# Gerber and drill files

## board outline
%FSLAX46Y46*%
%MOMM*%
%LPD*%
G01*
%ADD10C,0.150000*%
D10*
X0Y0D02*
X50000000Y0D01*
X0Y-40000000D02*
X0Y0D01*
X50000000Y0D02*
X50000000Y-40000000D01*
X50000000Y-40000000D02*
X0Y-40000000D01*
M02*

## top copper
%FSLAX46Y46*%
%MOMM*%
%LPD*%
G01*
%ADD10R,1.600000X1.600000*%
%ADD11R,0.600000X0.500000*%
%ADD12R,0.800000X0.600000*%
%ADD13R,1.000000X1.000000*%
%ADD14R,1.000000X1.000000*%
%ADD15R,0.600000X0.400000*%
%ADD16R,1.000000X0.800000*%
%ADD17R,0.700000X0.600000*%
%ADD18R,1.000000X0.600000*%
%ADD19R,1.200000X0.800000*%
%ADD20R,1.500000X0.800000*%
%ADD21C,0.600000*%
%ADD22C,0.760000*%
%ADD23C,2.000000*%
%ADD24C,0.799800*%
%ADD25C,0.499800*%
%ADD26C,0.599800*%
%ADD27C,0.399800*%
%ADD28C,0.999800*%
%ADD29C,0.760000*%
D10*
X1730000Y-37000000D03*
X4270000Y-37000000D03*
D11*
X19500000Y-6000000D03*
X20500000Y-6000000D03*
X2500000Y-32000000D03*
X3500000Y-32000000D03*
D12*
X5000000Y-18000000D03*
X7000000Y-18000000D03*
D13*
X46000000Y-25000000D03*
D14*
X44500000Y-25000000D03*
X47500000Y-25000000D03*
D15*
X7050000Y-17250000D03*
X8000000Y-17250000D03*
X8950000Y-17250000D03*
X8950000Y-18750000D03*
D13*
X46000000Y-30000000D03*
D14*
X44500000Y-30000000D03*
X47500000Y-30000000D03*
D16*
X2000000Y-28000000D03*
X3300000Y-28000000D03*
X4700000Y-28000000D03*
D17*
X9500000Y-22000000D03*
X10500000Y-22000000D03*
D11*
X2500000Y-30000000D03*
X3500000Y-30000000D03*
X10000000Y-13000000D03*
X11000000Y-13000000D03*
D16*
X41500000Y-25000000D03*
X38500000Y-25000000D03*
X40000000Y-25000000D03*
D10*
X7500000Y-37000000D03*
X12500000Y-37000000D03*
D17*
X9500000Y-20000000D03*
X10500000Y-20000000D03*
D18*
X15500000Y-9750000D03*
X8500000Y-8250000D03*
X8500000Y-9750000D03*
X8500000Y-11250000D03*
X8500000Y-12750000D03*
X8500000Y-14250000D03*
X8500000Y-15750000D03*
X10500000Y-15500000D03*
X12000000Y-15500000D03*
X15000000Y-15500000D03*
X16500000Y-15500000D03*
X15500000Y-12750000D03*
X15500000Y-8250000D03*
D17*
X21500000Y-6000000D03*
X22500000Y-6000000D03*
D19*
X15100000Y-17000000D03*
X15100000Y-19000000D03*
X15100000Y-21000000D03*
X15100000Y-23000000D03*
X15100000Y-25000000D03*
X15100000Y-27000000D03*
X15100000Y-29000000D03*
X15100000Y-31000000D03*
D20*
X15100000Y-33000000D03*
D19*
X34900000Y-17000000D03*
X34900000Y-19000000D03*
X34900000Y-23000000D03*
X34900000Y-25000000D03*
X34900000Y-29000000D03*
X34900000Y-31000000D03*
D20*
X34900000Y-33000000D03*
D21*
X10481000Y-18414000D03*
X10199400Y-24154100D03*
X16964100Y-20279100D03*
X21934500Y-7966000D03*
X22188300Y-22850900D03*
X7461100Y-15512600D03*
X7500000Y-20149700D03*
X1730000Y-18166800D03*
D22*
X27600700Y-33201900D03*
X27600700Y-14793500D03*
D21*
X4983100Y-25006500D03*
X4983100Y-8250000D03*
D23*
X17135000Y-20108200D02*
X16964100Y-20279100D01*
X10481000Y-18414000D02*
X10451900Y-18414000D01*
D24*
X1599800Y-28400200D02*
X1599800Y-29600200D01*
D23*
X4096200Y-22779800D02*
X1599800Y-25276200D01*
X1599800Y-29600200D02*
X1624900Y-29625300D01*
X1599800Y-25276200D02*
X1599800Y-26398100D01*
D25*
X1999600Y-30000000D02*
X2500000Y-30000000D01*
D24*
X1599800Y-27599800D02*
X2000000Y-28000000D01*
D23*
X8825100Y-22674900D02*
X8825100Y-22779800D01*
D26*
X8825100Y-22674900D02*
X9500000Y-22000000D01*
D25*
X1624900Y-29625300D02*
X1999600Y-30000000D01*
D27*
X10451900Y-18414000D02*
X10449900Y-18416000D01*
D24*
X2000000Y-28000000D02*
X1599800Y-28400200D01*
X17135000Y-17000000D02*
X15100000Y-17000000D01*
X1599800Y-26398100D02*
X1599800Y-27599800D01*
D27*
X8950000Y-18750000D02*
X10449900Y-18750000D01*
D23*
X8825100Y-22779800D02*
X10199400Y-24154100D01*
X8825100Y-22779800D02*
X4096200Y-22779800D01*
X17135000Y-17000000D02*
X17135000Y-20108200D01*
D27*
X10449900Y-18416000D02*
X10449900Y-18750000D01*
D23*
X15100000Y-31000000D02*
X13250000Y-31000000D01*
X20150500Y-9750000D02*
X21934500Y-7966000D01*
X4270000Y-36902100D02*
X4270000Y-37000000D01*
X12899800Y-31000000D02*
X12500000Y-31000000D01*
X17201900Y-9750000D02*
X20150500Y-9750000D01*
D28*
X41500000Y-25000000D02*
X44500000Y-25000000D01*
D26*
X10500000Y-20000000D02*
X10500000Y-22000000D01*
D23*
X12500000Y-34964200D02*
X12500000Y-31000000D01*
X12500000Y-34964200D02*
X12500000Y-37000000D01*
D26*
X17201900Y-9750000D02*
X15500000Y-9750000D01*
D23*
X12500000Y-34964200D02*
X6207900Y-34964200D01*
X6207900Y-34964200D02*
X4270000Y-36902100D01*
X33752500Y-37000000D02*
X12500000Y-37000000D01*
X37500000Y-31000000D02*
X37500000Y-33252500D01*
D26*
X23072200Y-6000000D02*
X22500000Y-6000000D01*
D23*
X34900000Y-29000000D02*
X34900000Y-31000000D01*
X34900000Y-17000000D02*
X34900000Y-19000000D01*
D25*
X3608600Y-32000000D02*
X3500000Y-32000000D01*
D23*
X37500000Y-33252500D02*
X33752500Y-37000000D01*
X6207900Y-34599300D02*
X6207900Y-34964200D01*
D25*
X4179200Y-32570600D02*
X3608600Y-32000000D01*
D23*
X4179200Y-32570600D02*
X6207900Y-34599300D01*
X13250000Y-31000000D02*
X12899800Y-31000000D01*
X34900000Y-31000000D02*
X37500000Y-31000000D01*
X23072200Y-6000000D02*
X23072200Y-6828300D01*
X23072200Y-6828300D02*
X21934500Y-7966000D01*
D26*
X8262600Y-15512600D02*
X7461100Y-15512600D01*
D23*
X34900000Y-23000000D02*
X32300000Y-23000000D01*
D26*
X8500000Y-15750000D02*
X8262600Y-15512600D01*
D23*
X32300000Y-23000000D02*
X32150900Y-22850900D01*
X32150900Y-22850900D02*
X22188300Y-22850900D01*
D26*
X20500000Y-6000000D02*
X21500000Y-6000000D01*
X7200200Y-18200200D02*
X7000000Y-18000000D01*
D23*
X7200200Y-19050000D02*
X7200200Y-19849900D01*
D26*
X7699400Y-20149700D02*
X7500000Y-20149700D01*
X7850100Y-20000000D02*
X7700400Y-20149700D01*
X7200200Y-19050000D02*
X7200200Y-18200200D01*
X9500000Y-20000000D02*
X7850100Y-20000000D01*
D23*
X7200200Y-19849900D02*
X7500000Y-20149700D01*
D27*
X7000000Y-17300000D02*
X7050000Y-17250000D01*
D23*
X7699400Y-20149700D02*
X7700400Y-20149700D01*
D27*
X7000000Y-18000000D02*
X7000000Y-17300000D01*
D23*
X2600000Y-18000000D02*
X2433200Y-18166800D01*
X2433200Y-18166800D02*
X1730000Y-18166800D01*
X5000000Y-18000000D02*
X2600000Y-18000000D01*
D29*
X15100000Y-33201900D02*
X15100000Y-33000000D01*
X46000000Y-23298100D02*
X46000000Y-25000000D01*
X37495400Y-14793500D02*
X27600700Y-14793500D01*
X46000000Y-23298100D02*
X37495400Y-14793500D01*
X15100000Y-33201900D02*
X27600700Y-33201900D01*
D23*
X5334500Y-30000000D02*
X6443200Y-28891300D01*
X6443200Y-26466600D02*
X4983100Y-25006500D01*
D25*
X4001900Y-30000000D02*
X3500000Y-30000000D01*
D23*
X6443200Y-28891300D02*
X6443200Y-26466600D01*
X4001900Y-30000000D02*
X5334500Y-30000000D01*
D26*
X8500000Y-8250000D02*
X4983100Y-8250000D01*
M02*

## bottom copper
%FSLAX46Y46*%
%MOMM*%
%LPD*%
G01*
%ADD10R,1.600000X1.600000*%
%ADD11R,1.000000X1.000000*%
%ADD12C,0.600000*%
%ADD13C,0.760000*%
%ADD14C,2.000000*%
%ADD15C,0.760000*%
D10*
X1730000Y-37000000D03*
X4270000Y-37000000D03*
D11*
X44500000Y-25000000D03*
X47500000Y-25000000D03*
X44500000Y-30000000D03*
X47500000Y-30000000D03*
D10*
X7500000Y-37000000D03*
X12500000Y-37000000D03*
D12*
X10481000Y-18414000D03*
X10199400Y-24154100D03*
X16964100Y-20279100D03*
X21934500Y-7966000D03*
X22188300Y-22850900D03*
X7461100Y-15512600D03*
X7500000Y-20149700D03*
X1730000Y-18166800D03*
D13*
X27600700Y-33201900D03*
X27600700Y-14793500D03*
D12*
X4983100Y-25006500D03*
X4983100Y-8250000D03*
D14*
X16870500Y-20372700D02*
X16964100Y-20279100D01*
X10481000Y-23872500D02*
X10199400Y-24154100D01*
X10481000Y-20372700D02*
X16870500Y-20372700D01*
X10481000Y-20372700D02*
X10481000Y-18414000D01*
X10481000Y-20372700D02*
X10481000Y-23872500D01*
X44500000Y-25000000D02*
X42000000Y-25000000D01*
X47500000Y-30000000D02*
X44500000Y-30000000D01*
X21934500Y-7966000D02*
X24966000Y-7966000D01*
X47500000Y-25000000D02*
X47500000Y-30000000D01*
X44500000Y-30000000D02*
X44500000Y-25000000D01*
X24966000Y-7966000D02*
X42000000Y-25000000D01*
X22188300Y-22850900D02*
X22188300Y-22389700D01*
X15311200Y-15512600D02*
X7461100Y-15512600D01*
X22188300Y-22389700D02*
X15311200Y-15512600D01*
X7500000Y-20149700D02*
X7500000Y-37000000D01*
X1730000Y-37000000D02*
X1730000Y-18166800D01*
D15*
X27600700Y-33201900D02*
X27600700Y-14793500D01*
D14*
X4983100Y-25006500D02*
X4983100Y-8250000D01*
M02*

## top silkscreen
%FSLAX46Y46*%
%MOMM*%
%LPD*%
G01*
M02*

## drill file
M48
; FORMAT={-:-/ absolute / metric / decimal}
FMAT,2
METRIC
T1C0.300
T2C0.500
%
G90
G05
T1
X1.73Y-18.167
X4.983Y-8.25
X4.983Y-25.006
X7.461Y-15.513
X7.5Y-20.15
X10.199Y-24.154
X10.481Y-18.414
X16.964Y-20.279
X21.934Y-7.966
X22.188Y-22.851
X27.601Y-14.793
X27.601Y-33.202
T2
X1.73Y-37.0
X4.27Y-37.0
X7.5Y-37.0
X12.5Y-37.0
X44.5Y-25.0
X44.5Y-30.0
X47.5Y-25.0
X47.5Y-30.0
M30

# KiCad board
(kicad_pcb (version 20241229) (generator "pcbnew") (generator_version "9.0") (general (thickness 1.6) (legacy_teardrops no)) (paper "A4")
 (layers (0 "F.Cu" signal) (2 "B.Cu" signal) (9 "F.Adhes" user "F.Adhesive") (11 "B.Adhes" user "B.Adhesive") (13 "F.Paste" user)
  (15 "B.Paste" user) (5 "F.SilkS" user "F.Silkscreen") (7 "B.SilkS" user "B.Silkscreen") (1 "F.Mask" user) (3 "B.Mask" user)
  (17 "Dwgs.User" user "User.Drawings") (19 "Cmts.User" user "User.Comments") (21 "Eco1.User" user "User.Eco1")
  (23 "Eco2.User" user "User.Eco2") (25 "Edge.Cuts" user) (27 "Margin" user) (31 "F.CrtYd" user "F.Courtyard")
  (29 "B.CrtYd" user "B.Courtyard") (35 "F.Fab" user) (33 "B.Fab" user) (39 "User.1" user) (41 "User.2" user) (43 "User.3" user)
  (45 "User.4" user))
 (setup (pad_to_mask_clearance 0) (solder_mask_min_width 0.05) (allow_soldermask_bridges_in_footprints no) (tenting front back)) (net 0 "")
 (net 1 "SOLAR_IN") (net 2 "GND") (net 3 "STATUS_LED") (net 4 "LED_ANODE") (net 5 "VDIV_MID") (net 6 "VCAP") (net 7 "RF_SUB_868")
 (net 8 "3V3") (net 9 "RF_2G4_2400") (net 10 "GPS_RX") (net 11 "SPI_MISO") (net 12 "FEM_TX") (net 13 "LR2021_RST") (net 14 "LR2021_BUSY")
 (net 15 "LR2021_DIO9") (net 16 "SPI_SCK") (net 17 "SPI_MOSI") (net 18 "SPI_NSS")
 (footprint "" (layer "F.Cu") (at 3 37)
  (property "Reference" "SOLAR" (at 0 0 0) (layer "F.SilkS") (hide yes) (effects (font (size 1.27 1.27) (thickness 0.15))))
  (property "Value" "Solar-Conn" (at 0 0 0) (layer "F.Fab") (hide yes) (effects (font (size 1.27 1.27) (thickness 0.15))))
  (pad "1" thru_hole rect (at -1.27 0) (size 1.6 1.6) (drill 0.5) (layers "*.Cu" "*.Mask") (remove_unused_layers no) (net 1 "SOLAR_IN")
   (thermal_bridge_angle 45))
  (pad "2" thru_hole rect (at 1.27 0) (size 1.6 1.6) (drill 0.5) (layers "*.Cu" "*.Mask") (remove_unused_layers no) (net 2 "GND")
   (thermal_bridge_angle 45)))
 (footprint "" (layer "F.Cu") (at 20 6)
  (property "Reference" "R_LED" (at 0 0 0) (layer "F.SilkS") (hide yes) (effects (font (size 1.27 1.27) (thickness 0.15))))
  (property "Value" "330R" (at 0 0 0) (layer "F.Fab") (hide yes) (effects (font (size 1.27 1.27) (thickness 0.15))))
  (pad "1" smd rect (at -0.5 0) (size 0.6 0.5) (layers "F.Cu" "F.Mask") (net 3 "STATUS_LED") (thermal_bridge_angle 45))
  (pad "2" smd rect (at 0.5 0) (size 0.6 0.5) (layers "F.Cu" "F.Mask") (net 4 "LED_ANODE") (thermal_bridge_angle 45)))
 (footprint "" (layer "F.Cu") (at 3 32)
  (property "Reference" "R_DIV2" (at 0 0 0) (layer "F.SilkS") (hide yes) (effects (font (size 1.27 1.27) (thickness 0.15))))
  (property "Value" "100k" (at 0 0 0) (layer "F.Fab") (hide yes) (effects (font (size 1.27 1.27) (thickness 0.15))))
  (pad "1" smd rect (at -0.5 0) (size 0.6 0.5) (layers "F.Cu" "F.Mask") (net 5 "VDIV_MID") (thermal_bridge_angle 45))
  (pad "2" smd rect (at 0.5 0) (size 0.6 0.5) (layers "F.Cu" "F.Mask") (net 2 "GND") (thermal_bridge_angle 45)))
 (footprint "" (layer "F.Cu") (at 6 18)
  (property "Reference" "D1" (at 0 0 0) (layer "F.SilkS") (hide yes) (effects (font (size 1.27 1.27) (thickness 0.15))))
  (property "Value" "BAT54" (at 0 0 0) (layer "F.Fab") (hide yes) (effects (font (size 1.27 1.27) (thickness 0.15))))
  (pad "A" smd rect (at -1 0) (size 0.8 0.6) (layers "F.Cu" "F.Mask") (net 1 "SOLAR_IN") (thermal_bridge_angle 45))
  (pad "K" smd rect (at 1 0) (size 0.8 0.6) (layers "F.Cu" "F.Mask") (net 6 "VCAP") (thermal_bridge_angle 45)))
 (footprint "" (layer "F.Cu") (at 46 25)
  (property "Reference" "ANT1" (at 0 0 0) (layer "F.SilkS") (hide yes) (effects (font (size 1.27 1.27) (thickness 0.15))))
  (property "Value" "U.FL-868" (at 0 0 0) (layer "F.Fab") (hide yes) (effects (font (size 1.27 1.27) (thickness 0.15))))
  (pad "1" smd rect (at 0 0) (size 1 1) (layers "F.Cu" "F.Mask") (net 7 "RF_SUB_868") (thermal_bridge_angle 45))
  (pad "2" thru_hole rect (at -1.5 0) (size 1 1) (drill 0.5) (layers "*.Cu" "*.Mask") (remove_unused_layers no) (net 2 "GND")
   (thermal_bridge_angle 45))
  (pad "3" thru_hole rect (at 1.5 0) (size 1 1) (drill 0.5) (layers "*.Cu" "*.Mask") (remove_unused_layers no) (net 2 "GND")
   (thermal_bridge_angle 45)))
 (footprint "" (layer "F.Cu") (at 8 18)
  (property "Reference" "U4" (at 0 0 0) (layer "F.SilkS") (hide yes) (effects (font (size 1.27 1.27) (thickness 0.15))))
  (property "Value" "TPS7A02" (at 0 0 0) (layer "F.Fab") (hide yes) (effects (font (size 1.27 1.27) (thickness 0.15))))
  (pad "1" smd rect (at -0.95 -0.75) (size 0.6 0.4) (layers "F.Cu" "F.Mask") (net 6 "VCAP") (thermal_bridge_angle 45))
  (pad "2" smd rect (at 0 -0.75) (size 0.6 0.4) (layers "F.Cu" "F.Mask") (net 2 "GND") (thermal_bridge_angle 45))
  (pad "3" smd rect (at 0.95 -0.75) (size 0.6 0.4) (layers "F.Cu" "F.Mask") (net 6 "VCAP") (thermal_bridge_angle 45))
  (pad "4" smd rect (at 0.95 0.75) (size 0.6 0.4) (layers "F.Cu" "F.Mask") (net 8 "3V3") (thermal_bridge_angle 45)))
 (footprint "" (layer "F.Cu") (at 46 30)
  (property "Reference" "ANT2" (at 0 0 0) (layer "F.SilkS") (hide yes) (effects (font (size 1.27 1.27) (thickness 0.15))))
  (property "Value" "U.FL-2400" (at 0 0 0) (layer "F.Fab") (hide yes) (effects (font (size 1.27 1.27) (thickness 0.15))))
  (pad "1" smd rect (at 0 0) (size 1 1) (layers "F.Cu" "F.Mask") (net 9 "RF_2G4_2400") (thermal_bridge_angle 45))
  (pad "2" thru_hole rect (at -1.5 0) (size 1 1) (drill 0.5) (layers "*.Cu" "*.Mask") (remove_unused_layers no) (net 2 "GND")
   (thermal_bridge_angle 45))
  (pad "3" thru_hole rect (at 1.5 0) (size 1 1) (drill 0.5) (layers "*.Cu" "*.Mask") (remove_unused_layers no) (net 2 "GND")
   (thermal_bridge_angle 45)))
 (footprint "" (layer "F.Cu") (at 4 28)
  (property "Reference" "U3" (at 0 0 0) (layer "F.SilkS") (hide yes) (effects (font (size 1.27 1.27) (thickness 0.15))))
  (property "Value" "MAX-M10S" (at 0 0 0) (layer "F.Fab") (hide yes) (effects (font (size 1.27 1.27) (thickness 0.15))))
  (pad "1" smd rect (at -2 0) (size 1 0.8) (layers "F.Cu" "F.Mask") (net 8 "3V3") (thermal_bridge_angle 45))
  (pad "2" smd rect (at -0.7 0) (size 1 0.8) (layers "F.Cu" "F.Mask") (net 2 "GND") (thermal_bridge_angle 45))
  (pad "3" smd rect (at 0.7 0) (size 1 0.8) (layers "F.Cu" "F.Mask") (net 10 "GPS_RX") (thermal_bridge_angle 45)))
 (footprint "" (layer "F.Cu") (at 10 22)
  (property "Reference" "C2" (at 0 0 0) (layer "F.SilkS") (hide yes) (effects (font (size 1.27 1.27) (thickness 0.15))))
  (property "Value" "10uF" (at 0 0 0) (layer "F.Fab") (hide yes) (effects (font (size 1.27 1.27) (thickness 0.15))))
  (pad "1" smd rect (at -0.5 0) (size 0.7 0.6) (layers "F.Cu" "F.Mask") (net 8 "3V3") (thermal_bridge_angle 45))
  (pad "2" smd rect (at 0.5 0) (size 0.7 0.6) (layers "F.Cu" "F.Mask") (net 2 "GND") (thermal_bridge_angle 45)))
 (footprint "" (layer "F.Cu") (at 3 30)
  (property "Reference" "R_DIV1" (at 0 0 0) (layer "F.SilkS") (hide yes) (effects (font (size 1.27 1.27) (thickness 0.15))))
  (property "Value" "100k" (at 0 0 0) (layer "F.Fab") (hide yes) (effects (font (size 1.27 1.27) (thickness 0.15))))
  (pad "1" smd rect (at -0.5 0) (size 0.6 0.5) (layers "F.Cu" "F.Mask") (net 8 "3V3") (thermal_bridge_angle 45))
  (pad "2" smd rect (at 0.5 0) (size 0.6 0.5) (layers "F.Cu" "F.Mask") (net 5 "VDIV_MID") (thermal_bridge_angle 45)))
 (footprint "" (layer "F.Cu") (at 10.5 13)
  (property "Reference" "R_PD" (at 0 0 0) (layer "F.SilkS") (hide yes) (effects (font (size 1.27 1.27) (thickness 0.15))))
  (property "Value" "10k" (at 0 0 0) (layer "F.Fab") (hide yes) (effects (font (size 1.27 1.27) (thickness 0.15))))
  (pad "1" smd rect (at -0.5 0) (size 0.6 0.5) (layers "F.Cu" "F.Mask") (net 2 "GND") (thermal_bridge_angle 45))
  (pad "2" smd rect (at 0.5 0) (size 0.6 0.5) (layers "F.Cu" "F.Mask") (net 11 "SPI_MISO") (thermal_bridge_angle 45)))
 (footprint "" (layer "F.Cu") (at 40 25)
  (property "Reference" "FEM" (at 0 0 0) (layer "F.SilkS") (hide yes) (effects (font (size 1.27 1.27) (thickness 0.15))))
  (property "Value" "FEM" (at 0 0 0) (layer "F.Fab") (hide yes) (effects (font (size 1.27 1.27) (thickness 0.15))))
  (pad "GND" smd rect (at 1.5 0) (size 1 0.8) (layers "F.Cu" "F.Mask") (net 2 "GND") (thermal_bridge_angle 45))
  (pad "TX" smd rect (at -1.5 0) (size 1 0.8) (layers "F.Cu" "F.Mask") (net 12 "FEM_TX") (thermal_bridge_angle 45))
  (pad "VCC" smd rect (at 0 0) (size 1 0.8) (layers "F.Cu" "F.Mask") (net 8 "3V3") (thermal_bridge_angle 45)))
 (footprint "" (layer "F.Cu") (at 10 37)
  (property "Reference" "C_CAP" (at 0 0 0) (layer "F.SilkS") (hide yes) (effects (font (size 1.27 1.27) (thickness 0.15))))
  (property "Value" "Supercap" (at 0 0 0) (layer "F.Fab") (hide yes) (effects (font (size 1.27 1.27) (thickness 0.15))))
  (pad "1" thru_hole rect (at -2.5 0) (size 1.6 1.6) (drill 0.5) (layers "*.Cu" "*.Mask") (remove_unused_layers no) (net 6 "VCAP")
   (thermal_bridge_angle 45))
  (pad "2" thru_hole rect (at 2.5 0) (size 1.6 1.6) (drill 0.5) (layers "*.Cu" "*.Mask") (remove_unused_layers no) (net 2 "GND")
   (thermal_bridge_angle 45)))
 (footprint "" (layer "F.Cu") (at 10 20)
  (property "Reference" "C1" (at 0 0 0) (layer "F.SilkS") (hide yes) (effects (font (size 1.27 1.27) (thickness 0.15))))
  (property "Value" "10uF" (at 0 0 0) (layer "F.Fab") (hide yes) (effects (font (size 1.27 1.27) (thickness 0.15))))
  (pad "1" smd rect (at -0.5 0) (size 0.7 0.6) (layers "F.Cu" "F.Mask") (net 6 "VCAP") (thermal_bridge_angle 45))
  (pad "2" smd rect (at 0.5 0) (size 0.7 0.6) (layers "F.Cu" "F.Mask") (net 2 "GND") (thermal_bridge_angle 45)))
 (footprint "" (layer "F.Cu") (at 12 12)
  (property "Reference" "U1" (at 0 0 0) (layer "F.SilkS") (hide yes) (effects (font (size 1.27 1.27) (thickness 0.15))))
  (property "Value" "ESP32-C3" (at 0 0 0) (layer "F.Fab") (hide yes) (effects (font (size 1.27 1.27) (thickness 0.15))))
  (pad "GND" smd rect (at 3.5 -2.25) (size 1 0.6) (layers "F.Cu" "F.Mask") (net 2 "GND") (thermal_bridge_angle 45))
  (pad "GPIO0" smd rect (at -3.5 -3.75) (size 1 0.6) (layers "F.Cu" "F.Mask") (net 5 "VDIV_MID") (thermal_bridge_angle 45))
  (pad "GPIO1" smd rect (at -3.5 -2.25) (size 1 0.6) (layers "F.Cu" "F.Mask") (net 10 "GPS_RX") (thermal_bridge_angle 45))
  (pad "GPIO2" smd rect (at -3.5 -0.75) (size 1 0.6) (layers "F.Cu" "F.Mask") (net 11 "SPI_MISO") (thermal_bridge_angle 45))
  (pad "GPIO3" smd rect (at -3.5 0.75) (size 1 0.6) (layers "F.Cu" "F.Mask") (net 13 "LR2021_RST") (thermal_bridge_angle 45))
  (pad "GPIO4" smd rect (at -3.5 2.25) (size 1 0.6) (layers "F.Cu" "F.Mask") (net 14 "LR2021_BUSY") (thermal_bridge_angle 45))
  (pad "GPIO5" smd rect (at -3.5 3.75) (size 1 0.6) (layers "F.Cu" "F.Mask") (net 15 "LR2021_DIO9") (thermal_bridge_angle 45))
  (pad "GPIO6" smd rect (at -1.5 3.5) (size 1 0.6) (layers "F.Cu" "F.Mask") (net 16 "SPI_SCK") (thermal_bridge_angle 45))
  (pad "GPIO7" smd rect (at 0 3.5) (size 1 0.6) (layers "F.Cu" "F.Mask") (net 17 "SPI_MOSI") (thermal_bridge_angle 45))
  (pad "GPIO9" smd rect (at 3 3.5) (size 1 0.6) (layers "F.Cu" "F.Mask") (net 3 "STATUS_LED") (thermal_bridge_angle 45))
  (pad "GPIO10" smd rect (at 4.5 3.5) (size 1 0.6) (layers "F.Cu" "F.Mask") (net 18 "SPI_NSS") (thermal_bridge_angle 45))
  (pad "GPIO19" smd rect (at 3.5 0.75) (size 1 0.6) (layers "F.Cu" "F.Mask") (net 12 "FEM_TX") (thermal_bridge_angle 45))
  (pad "VCC" smd rect (at 3.5 -3.75) (size 1 0.6) (layers "F.Cu" "F.Mask") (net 8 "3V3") (thermal_bridge_angle 45)))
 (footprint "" (layer "F.Cu") (at 22 6)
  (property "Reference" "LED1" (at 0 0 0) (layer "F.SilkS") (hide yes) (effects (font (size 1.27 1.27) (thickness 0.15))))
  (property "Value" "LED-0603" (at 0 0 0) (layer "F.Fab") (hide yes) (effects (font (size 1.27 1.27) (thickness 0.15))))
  (pad "A" smd rect (at -0.5 0) (size 0.7 0.6) (layers "F.Cu" "F.Mask") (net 4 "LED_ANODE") (thermal_bridge_angle 45))
  (pad "K" smd rect (at 0.5 0) (size 0.7 0.6) (layers "F.Cu" "F.Mask") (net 2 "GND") (thermal_bridge_angle 45)))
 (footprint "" (layer "F.Cu") (at 25 25)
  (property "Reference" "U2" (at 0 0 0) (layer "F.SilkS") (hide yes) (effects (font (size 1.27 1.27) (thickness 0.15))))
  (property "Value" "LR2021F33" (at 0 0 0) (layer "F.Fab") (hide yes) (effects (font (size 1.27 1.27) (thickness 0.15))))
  (pad "1" smd rect (at -9.9 -8) (size 1.2 0.8) (layers "F.Cu" "F.Mask") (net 8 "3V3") (thermal_bridge_angle 45))
  (pad "2" smd rect (at -9.9 -6) (size 1.2 0.8) (layers "F.Cu" "F.Mask") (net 2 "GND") (thermal_bridge_angle 45))
  (pad "3" smd rect (at -9.9 -4) (size 1.2 0.8) (layers "F.Cu" "F.Mask") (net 11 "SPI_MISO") (thermal_bridge_angle 45))
  (pad "4" smd rect (at -9.9 -2) (size 1.2 0.8) (layers "F.Cu" "F.Mask") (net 17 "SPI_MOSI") (thermal_bridge_angle 45))
  (pad "5" smd rect (at -9.9 0) (size 1.2 0.8) (layers "F.Cu" "F.Mask") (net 16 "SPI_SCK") (thermal_bridge_angle 45))
  (pad "6" smd rect (at -9.9 2) (size 1.2 0.8) (layers "F.Cu" "F.Mask") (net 18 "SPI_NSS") (thermal_bridge_angle 45))
  (pad "7" smd rect (at -9.9 4) (size 1.2 0.8) (layers "F.Cu" "F.Mask") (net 14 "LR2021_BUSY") (thermal_bridge_angle 45))
  (pad "8" smd rect (at -9.9 6) (size 1.2 0.8) (layers "F.Cu" "F.Mask") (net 2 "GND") (thermal_bridge_angle 45))
  (pad "9" smd rect (at -9.9 8) (size 1.5 0.8) (layers "F.Cu" "F.Mask") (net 7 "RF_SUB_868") (thermal_bridge_angle 45))
  (pad "10" smd rect (at 9.9 -8) (size 1.2 0.8) (layers "F.Cu" "F.Mask") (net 2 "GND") (thermal_bridge_angle 45))
  (pad "11" smd rect (at 9.9 -6) (size 1.2 0.8) (layers "F.Cu" "F.Mask") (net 2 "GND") (thermal_bridge_angle 45))
  (pad "13" smd rect (at 9.9 -2) (size 1.2 0.8) (layers "F.Cu" "F.Mask") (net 15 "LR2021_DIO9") (thermal_bridge_angle 45))
  (pad "14" smd rect (at 9.9 0) (size 1.2 0.8) (layers "F.Cu" "F.Mask") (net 13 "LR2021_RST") (thermal_bridge_angle 45))
  (pad "16" smd rect (at 9.9 4) (size 1.2 0.8) (layers "F.Cu" "F.Mask") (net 2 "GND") (thermal_bridge_angle 45))
  (pad "17" smd rect (at 9.9 6) (size 1.2 0.8) (layers "F.Cu" "F.Mask") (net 2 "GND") (thermal_bridge_angle 45))
  (pad "18" smd rect (at 9.9 8) (size 1.5 0.8) (layers "F.Cu" "F.Mask") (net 9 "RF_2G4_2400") (thermal_bridge_angle 45)))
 (gr_line (start 0 0) (end 50 0) (stroke (width 0.15) (type default)) (layer "Edge.Cuts"))
 (gr_line (start 0 40) (end 0 0) (stroke (width 0.15) (type default)) (layer "Edge.Cuts"))
 (gr_line (start 50 0) (end 50 40) (stroke (width 0.15) (type default)) (layer "Edge.Cuts"))
 (gr_line (start 50 40) (end 0 40) (stroke (width 0.15) (type default)) (layer "Edge.Cuts"))
 (segment (start 17.135 20.1082) (end 16.9641 20.2791) (width 2) (layer "F.Cu") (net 8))
 (segment (start 10.481 18.414) (end 10.4519 18.414) (width 2) (layer "F.Cu") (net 8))
 (segment (start 1.5998 28.4002) (end 1.5998 29.6002) (width 0.7998) (layer "F.Cu") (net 8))
 (segment (start 4.0962 22.7798) (end 1.5998 25.2762) (width 2) (layer "F.Cu") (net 8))
 (segment (start 1.5998 29.6002) (end 1.6249 29.6253) (width 2) (layer "F.Cu") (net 8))
 (segment (start 1.5998 25.2762) (end 1.5998 26.3981) (width 2) (layer "F.Cu") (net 8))
 (segment (start 1.9996 30) (end 2.5 30) (width 0.4998) (layer "F.Cu") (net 8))
 (segment (start 1.5998 27.5998) (end 2 28) (width 0.7998) (layer "F.Cu") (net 8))
 (segment (start 8.8251 22.6749) (end 8.8251 22.7798) (width 2) (layer "F.Cu") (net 8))
 (segment (start 8.8251 22.6749) (end 9.5 22) (width 0.5998) (layer "F.Cu") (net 8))
 (segment (start 1.6249 29.6253) (end 1.9996 30) (width 0.4998) (layer "F.Cu") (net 8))
 (segment (start 10.4519 18.414) (end 10.4499 18.416) (width 0.3998) (layer "F.Cu") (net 8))
 (segment (start 2 28) (end 1.5998 28.4002) (width 0.7998) (layer "F.Cu") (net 8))
 (segment (start 17.135 17) (end 15.1 17) (width 0.7998) (layer "F.Cu") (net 8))
 (segment (start 1.5998 26.3981) (end 1.5998 27.5998) (width 0.7998) (layer "F.Cu") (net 8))
 (segment (start 8.95 18.75) (end 10.4499 18.75) (width 0.3998) (layer "F.Cu") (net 8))
 (segment (start 8.8251 22.7798) (end 10.1994 24.1541) (width 2) (layer "F.Cu") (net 8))
 (segment (start 8.8251 22.7798) (end 4.0962 22.7798) (width 2) (layer "F.Cu") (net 8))
 (segment (start 17.135 17) (end 17.135 20.1082) (width 2) (layer "F.Cu") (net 8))
 (segment (start 10.4499 18.416) (end 10.4499 18.75) (width 0.3998) (layer "F.Cu") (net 8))
 (via (at 10.481 18.414) (size 0.6) (drill 0.3) (layers "F.Cu" "B.Cu") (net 8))
 (via (at 10.1994 24.1541) (size 0.6) (drill 0.3) (layers "F.Cu" "B.Cu") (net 8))
 (via (at 16.9641 20.2791) (size 0.6) (drill 0.3) (layers "F.Cu" "B.Cu") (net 8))
 (segment (start 16.8705 20.3727) (end 16.9641 20.2791) (width 2) (layer "B.Cu") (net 8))
 (segment (start 10.481 23.8725) (end 10.1994 24.1541) (width 2) (layer "B.Cu") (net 8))
 (segment (start 10.481 20.3727) (end 16.8705 20.3727) (width 2) (layer "B.Cu") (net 8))
 (segment (start 10.481 20.3727) (end 10.481 18.414) (width 2) (layer "B.Cu") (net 8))
 (segment (start 10.481 20.3727) (end 10.481 23.8725) (width 2) (layer "B.Cu") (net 8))
 (segment (start 15.1 31) (end 13.25 31) (width 2) (layer "F.Cu") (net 2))
 (segment (start 20.1505 9.75) (end 21.9345 7.966) (width 2) (layer "F.Cu") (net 2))
 (segment (start 4.27 36.9021) (end 4.27 37) (width 2) (layer "F.Cu") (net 2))
 (segment (start 12.8998 31) (end 12.5 31) (width 2) (layer "F.Cu") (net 2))
 (segment (start 17.2019 9.75) (end 20.1505 9.75) (width 2) (layer "F.Cu") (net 2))
 (segment (start 41.5 25) (end 44.5 25) (width 0.9998) (layer "F.Cu") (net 2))
 (segment (start 10.5 20) (end 10.5 22) (width 0.5998) (layer "F.Cu") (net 2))
 (segment (start 12.5 34.9642) (end 12.5 31) (width 2) (layer "F.Cu") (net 2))
 (segment (start 12.5 34.9642) (end 12.5 37) (width 2) (layer "F.Cu") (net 2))
 (segment (start 17.2019 9.75) (end 15.5 9.75) (width 0.5998) (layer "F.Cu") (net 2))
 (segment (start 12.5 34.9642) (end 6.2079 34.9642) (width 2) (layer "F.Cu") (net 2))
 (segment (start 6.2079 34.9642) (end 4.27 36.9021) (width 2) (layer "F.Cu") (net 2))
 (segment (start 33.7525 37) (end 12.5 37) (width 2) (layer "F.Cu") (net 2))
 (segment (start 37.5 31) (end 37.5 33.2525) (width 2) (layer "F.Cu") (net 2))
 (segment (start 23.0722 6) (end 22.5 6) (width 0.5998) (layer "F.Cu") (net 2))
 (segment (start 34.9 29) (end 34.9 31) (width 2) (layer "F.Cu") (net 2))
 (segment (start 34.9 17) (end 34.9 19) (width 2) (layer "F.Cu") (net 2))
 (segment (start 3.6086 32) (end 3.5 32) (width 0.4998) (layer "F.Cu") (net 2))
 (segment (start 37.5 33.2525) (end 33.7525 37) (width 2) (layer "F.Cu") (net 2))
 (segment (start 6.2079 34.5993) (end 6.2079 34.9642) (width 2) (layer "F.Cu") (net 2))
 (segment (start 4.1792 32.5706) (end 3.6086 32) (width 0.4998) (layer "F.Cu") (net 2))
 (segment (start 4.1792 32.5706) (end 6.2079 34.5993) (width 2) (layer "F.Cu") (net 2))
 (segment (start 13.25 31) (end 12.8998 31) (width 2) (layer "F.Cu") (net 2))
 (segment (start 34.9 31) (end 37.5 31) (width 2) (layer "F.Cu") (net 2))
 (segment (start 23.0722 6) (end 23.0722 6.8283) (width 2) (layer "F.Cu") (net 2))
 (segment (start 23.0722 6.8283) (end 21.9345 7.966) (width 2) (layer "F.Cu") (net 2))
 (via (at 21.9345 7.966) (size 0.6) (drill 0.3) (layers "F.Cu" "B.Cu") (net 2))
 (segment (start 44.5 25) (end 42 25) (width 2) (layer "B.Cu") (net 2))
 (segment (start 47.5 30) (end 44.5 30) (width 2) (layer "B.Cu") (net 2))
 (segment (start 21.9345 7.966) (end 24.966 7.966) (width 2) (layer "B.Cu") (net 2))
 (segment (start 47.5 25) (end 47.5 30) (width 2) (layer "B.Cu") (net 2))
 (segment (start 44.5 30) (end 44.5 25) (width 2) (layer "B.Cu") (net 2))
 (segment (start 24.966 7.966) (end 42 25) (width 2) (layer "B.Cu") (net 2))
 (segment (start 8.2626 15.5126) (end 7.4611 15.5126) (width 0.5998) (layer "F.Cu") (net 15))
 (segment (start 34.9 23) (end 32.3 23) (width 2) (layer "F.Cu") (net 15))
 (segment (start 8.5 15.75) (end 8.2626 15.5126) (width 0.5998) (layer "F.Cu") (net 15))
 (segment (start 32.3 23) (end 32.1509 22.8509) (width 2) (layer "F.Cu") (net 15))
 (segment (start 32.1509 22.8509) (end 22.1883 22.8509) (width 2) (layer "F.Cu") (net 15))
 (via (at 22.1883 22.8509) (size 0.6) (drill 0.3) (layers "F.Cu" "B.Cu") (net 15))
 (via (at 7.4611 15.5126) (size 0.6) (drill 0.3) (layers "F.Cu" "B.Cu") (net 15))
 (segment (start 22.1883 22.8509) (end 22.1883 22.3897) (width 2) (layer "B.Cu") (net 15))
 (segment (start 15.3112 15.5126) (end 7.4611 15.5126) (width 2) (layer "B.Cu") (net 15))
 (segment (start 22.1883 22.3897) (end 15.3112 15.5126) (width 2) (layer "B.Cu") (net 15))
 (segment (start 20.5 6) (end 21.5 6) (width 0.5998) (layer "F.Cu") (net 4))
 (segment (start 7.2002 18.2002) (end 7 18) (width 0.5998) (layer "F.Cu") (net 6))
 (segment (start 7.2002 19.05) (end 7.2002 19.8499) (width 2) (layer "F.Cu") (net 6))
 (segment (start 7.6994 20.1497) (end 7.5 20.1497) (width 0.5998) (layer "F.Cu") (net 6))
 (segment (start 7.8501 20) (end 7.7004 20.1497) (width 0.5998) (layer "F.Cu") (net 6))
 (segment (start 7.2002 19.05) (end 7.2002 18.2002) (width 0.5998) (layer "F.Cu") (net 6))
 (segment (start 9.5 20) (end 7.8501 20) (width 0.5998) (layer "F.Cu") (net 6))
 (segment (start 7.2002 19.8499) (end 7.5 20.1497) (width 2) (layer "F.Cu") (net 6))
 (segment (start 7 17.3) (end 7.05 17.25) (width 0.3998) (layer "F.Cu") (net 6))
 (segment (start 7.6994 20.1497) (end 7.7004 20.1497) (width 2) (layer "F.Cu") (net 6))
 (segment (start 7 18) (end 7 17.3) (width 0.3998) (layer "F.Cu") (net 6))
 (via (at 7.5 20.1497) (size 0.6) (drill 0.3) (layers "F.Cu" "B.Cu") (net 6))
 (segment (start 7.5 20.1497) (end 7.5 37) (width 2) (layer "B.Cu") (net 6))
 (segment (start 2.6 18) (end 2.4332 18.1668) (width 2) (layer "F.Cu") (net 1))
 (segment (start 2.4332 18.1668) (end 1.73 18.1668) (width 2) (layer "F.Cu") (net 1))
 (segment (start 5 18) (end 2.6 18) (width 2) (layer "F.Cu") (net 1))
 (via (at 1.73 18.1668) (size 0.6) (drill 0.3) (layers "F.Cu" "B.Cu") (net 1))
 (segment (start 1.73 37) (end 1.73 18.1668) (width 2) (layer "B.Cu") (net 1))
 (segment (start 15.1 33.2019) (end 15.1 33) (width 0.76) (layer "F.Cu") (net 7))
 (segment (start 46 23.2981) (end 46 25) (width 0.76) (layer "F.Cu") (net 7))
 (segment (start 37.4954 14.7935) (end 27.6007 14.7935) (width 0.76) (layer "F.Cu") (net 7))
 (segment (start 46 23.2981) (end 37.4954 14.7935) (width 0.76) (layer "F.Cu") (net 7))
 (segment (start 15.1 33.2019) (end 27.6007 33.2019) (width 0.76) (layer "F.Cu") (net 7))
 (via (at 27.6007 33.2019) (size 0.76) (drill 0.3) (layers "F.Cu" "B.Cu") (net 7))
 (via (at 27.6007 14.7935) (size 0.76) (drill 0.3) (layers "F.Cu" "B.Cu") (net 7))
 (segment (start 27.6007 33.2019) (end 27.6007 14.7935) (width 0.76) (layer "B.Cu") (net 7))
 (segment (start 5.3345 30) (end 6.4432 28.8913) (width 2) (layer "F.Cu") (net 5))
 (segment (start 6.4432 26.4666) (end 4.9831 25.0065) (width 2) (layer "F.Cu") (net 5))
 (segment (start 4.0019 30) (end 3.5 30) (width 0.4998) (layer "F.Cu") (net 5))
 (segment (start 6.4432 28.8913) (end 6.4432 26.4666) (width 2) (layer "F.Cu") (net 5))
 (segment (start 4.0019 30) (end 5.3345 30) (width 2) (layer "F.Cu") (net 5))
 (segment (start 8.5 8.25) (end 4.9831 8.25) (width 0.5998) (layer "F.Cu") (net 5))
 (via (at 4.9831 25.0065) (size 0.6) (drill 0.3) (layers "F.Cu" "B.Cu") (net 5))
 (via (at 4.9831 8.25) (size 0.6) (drill 0.3) (layers "F.Cu" "B.Cu") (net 5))
 (segment (start 4.9831 25.0065) (end 4.9831 8.25) (width 2) (layer "B.Cu") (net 5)))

